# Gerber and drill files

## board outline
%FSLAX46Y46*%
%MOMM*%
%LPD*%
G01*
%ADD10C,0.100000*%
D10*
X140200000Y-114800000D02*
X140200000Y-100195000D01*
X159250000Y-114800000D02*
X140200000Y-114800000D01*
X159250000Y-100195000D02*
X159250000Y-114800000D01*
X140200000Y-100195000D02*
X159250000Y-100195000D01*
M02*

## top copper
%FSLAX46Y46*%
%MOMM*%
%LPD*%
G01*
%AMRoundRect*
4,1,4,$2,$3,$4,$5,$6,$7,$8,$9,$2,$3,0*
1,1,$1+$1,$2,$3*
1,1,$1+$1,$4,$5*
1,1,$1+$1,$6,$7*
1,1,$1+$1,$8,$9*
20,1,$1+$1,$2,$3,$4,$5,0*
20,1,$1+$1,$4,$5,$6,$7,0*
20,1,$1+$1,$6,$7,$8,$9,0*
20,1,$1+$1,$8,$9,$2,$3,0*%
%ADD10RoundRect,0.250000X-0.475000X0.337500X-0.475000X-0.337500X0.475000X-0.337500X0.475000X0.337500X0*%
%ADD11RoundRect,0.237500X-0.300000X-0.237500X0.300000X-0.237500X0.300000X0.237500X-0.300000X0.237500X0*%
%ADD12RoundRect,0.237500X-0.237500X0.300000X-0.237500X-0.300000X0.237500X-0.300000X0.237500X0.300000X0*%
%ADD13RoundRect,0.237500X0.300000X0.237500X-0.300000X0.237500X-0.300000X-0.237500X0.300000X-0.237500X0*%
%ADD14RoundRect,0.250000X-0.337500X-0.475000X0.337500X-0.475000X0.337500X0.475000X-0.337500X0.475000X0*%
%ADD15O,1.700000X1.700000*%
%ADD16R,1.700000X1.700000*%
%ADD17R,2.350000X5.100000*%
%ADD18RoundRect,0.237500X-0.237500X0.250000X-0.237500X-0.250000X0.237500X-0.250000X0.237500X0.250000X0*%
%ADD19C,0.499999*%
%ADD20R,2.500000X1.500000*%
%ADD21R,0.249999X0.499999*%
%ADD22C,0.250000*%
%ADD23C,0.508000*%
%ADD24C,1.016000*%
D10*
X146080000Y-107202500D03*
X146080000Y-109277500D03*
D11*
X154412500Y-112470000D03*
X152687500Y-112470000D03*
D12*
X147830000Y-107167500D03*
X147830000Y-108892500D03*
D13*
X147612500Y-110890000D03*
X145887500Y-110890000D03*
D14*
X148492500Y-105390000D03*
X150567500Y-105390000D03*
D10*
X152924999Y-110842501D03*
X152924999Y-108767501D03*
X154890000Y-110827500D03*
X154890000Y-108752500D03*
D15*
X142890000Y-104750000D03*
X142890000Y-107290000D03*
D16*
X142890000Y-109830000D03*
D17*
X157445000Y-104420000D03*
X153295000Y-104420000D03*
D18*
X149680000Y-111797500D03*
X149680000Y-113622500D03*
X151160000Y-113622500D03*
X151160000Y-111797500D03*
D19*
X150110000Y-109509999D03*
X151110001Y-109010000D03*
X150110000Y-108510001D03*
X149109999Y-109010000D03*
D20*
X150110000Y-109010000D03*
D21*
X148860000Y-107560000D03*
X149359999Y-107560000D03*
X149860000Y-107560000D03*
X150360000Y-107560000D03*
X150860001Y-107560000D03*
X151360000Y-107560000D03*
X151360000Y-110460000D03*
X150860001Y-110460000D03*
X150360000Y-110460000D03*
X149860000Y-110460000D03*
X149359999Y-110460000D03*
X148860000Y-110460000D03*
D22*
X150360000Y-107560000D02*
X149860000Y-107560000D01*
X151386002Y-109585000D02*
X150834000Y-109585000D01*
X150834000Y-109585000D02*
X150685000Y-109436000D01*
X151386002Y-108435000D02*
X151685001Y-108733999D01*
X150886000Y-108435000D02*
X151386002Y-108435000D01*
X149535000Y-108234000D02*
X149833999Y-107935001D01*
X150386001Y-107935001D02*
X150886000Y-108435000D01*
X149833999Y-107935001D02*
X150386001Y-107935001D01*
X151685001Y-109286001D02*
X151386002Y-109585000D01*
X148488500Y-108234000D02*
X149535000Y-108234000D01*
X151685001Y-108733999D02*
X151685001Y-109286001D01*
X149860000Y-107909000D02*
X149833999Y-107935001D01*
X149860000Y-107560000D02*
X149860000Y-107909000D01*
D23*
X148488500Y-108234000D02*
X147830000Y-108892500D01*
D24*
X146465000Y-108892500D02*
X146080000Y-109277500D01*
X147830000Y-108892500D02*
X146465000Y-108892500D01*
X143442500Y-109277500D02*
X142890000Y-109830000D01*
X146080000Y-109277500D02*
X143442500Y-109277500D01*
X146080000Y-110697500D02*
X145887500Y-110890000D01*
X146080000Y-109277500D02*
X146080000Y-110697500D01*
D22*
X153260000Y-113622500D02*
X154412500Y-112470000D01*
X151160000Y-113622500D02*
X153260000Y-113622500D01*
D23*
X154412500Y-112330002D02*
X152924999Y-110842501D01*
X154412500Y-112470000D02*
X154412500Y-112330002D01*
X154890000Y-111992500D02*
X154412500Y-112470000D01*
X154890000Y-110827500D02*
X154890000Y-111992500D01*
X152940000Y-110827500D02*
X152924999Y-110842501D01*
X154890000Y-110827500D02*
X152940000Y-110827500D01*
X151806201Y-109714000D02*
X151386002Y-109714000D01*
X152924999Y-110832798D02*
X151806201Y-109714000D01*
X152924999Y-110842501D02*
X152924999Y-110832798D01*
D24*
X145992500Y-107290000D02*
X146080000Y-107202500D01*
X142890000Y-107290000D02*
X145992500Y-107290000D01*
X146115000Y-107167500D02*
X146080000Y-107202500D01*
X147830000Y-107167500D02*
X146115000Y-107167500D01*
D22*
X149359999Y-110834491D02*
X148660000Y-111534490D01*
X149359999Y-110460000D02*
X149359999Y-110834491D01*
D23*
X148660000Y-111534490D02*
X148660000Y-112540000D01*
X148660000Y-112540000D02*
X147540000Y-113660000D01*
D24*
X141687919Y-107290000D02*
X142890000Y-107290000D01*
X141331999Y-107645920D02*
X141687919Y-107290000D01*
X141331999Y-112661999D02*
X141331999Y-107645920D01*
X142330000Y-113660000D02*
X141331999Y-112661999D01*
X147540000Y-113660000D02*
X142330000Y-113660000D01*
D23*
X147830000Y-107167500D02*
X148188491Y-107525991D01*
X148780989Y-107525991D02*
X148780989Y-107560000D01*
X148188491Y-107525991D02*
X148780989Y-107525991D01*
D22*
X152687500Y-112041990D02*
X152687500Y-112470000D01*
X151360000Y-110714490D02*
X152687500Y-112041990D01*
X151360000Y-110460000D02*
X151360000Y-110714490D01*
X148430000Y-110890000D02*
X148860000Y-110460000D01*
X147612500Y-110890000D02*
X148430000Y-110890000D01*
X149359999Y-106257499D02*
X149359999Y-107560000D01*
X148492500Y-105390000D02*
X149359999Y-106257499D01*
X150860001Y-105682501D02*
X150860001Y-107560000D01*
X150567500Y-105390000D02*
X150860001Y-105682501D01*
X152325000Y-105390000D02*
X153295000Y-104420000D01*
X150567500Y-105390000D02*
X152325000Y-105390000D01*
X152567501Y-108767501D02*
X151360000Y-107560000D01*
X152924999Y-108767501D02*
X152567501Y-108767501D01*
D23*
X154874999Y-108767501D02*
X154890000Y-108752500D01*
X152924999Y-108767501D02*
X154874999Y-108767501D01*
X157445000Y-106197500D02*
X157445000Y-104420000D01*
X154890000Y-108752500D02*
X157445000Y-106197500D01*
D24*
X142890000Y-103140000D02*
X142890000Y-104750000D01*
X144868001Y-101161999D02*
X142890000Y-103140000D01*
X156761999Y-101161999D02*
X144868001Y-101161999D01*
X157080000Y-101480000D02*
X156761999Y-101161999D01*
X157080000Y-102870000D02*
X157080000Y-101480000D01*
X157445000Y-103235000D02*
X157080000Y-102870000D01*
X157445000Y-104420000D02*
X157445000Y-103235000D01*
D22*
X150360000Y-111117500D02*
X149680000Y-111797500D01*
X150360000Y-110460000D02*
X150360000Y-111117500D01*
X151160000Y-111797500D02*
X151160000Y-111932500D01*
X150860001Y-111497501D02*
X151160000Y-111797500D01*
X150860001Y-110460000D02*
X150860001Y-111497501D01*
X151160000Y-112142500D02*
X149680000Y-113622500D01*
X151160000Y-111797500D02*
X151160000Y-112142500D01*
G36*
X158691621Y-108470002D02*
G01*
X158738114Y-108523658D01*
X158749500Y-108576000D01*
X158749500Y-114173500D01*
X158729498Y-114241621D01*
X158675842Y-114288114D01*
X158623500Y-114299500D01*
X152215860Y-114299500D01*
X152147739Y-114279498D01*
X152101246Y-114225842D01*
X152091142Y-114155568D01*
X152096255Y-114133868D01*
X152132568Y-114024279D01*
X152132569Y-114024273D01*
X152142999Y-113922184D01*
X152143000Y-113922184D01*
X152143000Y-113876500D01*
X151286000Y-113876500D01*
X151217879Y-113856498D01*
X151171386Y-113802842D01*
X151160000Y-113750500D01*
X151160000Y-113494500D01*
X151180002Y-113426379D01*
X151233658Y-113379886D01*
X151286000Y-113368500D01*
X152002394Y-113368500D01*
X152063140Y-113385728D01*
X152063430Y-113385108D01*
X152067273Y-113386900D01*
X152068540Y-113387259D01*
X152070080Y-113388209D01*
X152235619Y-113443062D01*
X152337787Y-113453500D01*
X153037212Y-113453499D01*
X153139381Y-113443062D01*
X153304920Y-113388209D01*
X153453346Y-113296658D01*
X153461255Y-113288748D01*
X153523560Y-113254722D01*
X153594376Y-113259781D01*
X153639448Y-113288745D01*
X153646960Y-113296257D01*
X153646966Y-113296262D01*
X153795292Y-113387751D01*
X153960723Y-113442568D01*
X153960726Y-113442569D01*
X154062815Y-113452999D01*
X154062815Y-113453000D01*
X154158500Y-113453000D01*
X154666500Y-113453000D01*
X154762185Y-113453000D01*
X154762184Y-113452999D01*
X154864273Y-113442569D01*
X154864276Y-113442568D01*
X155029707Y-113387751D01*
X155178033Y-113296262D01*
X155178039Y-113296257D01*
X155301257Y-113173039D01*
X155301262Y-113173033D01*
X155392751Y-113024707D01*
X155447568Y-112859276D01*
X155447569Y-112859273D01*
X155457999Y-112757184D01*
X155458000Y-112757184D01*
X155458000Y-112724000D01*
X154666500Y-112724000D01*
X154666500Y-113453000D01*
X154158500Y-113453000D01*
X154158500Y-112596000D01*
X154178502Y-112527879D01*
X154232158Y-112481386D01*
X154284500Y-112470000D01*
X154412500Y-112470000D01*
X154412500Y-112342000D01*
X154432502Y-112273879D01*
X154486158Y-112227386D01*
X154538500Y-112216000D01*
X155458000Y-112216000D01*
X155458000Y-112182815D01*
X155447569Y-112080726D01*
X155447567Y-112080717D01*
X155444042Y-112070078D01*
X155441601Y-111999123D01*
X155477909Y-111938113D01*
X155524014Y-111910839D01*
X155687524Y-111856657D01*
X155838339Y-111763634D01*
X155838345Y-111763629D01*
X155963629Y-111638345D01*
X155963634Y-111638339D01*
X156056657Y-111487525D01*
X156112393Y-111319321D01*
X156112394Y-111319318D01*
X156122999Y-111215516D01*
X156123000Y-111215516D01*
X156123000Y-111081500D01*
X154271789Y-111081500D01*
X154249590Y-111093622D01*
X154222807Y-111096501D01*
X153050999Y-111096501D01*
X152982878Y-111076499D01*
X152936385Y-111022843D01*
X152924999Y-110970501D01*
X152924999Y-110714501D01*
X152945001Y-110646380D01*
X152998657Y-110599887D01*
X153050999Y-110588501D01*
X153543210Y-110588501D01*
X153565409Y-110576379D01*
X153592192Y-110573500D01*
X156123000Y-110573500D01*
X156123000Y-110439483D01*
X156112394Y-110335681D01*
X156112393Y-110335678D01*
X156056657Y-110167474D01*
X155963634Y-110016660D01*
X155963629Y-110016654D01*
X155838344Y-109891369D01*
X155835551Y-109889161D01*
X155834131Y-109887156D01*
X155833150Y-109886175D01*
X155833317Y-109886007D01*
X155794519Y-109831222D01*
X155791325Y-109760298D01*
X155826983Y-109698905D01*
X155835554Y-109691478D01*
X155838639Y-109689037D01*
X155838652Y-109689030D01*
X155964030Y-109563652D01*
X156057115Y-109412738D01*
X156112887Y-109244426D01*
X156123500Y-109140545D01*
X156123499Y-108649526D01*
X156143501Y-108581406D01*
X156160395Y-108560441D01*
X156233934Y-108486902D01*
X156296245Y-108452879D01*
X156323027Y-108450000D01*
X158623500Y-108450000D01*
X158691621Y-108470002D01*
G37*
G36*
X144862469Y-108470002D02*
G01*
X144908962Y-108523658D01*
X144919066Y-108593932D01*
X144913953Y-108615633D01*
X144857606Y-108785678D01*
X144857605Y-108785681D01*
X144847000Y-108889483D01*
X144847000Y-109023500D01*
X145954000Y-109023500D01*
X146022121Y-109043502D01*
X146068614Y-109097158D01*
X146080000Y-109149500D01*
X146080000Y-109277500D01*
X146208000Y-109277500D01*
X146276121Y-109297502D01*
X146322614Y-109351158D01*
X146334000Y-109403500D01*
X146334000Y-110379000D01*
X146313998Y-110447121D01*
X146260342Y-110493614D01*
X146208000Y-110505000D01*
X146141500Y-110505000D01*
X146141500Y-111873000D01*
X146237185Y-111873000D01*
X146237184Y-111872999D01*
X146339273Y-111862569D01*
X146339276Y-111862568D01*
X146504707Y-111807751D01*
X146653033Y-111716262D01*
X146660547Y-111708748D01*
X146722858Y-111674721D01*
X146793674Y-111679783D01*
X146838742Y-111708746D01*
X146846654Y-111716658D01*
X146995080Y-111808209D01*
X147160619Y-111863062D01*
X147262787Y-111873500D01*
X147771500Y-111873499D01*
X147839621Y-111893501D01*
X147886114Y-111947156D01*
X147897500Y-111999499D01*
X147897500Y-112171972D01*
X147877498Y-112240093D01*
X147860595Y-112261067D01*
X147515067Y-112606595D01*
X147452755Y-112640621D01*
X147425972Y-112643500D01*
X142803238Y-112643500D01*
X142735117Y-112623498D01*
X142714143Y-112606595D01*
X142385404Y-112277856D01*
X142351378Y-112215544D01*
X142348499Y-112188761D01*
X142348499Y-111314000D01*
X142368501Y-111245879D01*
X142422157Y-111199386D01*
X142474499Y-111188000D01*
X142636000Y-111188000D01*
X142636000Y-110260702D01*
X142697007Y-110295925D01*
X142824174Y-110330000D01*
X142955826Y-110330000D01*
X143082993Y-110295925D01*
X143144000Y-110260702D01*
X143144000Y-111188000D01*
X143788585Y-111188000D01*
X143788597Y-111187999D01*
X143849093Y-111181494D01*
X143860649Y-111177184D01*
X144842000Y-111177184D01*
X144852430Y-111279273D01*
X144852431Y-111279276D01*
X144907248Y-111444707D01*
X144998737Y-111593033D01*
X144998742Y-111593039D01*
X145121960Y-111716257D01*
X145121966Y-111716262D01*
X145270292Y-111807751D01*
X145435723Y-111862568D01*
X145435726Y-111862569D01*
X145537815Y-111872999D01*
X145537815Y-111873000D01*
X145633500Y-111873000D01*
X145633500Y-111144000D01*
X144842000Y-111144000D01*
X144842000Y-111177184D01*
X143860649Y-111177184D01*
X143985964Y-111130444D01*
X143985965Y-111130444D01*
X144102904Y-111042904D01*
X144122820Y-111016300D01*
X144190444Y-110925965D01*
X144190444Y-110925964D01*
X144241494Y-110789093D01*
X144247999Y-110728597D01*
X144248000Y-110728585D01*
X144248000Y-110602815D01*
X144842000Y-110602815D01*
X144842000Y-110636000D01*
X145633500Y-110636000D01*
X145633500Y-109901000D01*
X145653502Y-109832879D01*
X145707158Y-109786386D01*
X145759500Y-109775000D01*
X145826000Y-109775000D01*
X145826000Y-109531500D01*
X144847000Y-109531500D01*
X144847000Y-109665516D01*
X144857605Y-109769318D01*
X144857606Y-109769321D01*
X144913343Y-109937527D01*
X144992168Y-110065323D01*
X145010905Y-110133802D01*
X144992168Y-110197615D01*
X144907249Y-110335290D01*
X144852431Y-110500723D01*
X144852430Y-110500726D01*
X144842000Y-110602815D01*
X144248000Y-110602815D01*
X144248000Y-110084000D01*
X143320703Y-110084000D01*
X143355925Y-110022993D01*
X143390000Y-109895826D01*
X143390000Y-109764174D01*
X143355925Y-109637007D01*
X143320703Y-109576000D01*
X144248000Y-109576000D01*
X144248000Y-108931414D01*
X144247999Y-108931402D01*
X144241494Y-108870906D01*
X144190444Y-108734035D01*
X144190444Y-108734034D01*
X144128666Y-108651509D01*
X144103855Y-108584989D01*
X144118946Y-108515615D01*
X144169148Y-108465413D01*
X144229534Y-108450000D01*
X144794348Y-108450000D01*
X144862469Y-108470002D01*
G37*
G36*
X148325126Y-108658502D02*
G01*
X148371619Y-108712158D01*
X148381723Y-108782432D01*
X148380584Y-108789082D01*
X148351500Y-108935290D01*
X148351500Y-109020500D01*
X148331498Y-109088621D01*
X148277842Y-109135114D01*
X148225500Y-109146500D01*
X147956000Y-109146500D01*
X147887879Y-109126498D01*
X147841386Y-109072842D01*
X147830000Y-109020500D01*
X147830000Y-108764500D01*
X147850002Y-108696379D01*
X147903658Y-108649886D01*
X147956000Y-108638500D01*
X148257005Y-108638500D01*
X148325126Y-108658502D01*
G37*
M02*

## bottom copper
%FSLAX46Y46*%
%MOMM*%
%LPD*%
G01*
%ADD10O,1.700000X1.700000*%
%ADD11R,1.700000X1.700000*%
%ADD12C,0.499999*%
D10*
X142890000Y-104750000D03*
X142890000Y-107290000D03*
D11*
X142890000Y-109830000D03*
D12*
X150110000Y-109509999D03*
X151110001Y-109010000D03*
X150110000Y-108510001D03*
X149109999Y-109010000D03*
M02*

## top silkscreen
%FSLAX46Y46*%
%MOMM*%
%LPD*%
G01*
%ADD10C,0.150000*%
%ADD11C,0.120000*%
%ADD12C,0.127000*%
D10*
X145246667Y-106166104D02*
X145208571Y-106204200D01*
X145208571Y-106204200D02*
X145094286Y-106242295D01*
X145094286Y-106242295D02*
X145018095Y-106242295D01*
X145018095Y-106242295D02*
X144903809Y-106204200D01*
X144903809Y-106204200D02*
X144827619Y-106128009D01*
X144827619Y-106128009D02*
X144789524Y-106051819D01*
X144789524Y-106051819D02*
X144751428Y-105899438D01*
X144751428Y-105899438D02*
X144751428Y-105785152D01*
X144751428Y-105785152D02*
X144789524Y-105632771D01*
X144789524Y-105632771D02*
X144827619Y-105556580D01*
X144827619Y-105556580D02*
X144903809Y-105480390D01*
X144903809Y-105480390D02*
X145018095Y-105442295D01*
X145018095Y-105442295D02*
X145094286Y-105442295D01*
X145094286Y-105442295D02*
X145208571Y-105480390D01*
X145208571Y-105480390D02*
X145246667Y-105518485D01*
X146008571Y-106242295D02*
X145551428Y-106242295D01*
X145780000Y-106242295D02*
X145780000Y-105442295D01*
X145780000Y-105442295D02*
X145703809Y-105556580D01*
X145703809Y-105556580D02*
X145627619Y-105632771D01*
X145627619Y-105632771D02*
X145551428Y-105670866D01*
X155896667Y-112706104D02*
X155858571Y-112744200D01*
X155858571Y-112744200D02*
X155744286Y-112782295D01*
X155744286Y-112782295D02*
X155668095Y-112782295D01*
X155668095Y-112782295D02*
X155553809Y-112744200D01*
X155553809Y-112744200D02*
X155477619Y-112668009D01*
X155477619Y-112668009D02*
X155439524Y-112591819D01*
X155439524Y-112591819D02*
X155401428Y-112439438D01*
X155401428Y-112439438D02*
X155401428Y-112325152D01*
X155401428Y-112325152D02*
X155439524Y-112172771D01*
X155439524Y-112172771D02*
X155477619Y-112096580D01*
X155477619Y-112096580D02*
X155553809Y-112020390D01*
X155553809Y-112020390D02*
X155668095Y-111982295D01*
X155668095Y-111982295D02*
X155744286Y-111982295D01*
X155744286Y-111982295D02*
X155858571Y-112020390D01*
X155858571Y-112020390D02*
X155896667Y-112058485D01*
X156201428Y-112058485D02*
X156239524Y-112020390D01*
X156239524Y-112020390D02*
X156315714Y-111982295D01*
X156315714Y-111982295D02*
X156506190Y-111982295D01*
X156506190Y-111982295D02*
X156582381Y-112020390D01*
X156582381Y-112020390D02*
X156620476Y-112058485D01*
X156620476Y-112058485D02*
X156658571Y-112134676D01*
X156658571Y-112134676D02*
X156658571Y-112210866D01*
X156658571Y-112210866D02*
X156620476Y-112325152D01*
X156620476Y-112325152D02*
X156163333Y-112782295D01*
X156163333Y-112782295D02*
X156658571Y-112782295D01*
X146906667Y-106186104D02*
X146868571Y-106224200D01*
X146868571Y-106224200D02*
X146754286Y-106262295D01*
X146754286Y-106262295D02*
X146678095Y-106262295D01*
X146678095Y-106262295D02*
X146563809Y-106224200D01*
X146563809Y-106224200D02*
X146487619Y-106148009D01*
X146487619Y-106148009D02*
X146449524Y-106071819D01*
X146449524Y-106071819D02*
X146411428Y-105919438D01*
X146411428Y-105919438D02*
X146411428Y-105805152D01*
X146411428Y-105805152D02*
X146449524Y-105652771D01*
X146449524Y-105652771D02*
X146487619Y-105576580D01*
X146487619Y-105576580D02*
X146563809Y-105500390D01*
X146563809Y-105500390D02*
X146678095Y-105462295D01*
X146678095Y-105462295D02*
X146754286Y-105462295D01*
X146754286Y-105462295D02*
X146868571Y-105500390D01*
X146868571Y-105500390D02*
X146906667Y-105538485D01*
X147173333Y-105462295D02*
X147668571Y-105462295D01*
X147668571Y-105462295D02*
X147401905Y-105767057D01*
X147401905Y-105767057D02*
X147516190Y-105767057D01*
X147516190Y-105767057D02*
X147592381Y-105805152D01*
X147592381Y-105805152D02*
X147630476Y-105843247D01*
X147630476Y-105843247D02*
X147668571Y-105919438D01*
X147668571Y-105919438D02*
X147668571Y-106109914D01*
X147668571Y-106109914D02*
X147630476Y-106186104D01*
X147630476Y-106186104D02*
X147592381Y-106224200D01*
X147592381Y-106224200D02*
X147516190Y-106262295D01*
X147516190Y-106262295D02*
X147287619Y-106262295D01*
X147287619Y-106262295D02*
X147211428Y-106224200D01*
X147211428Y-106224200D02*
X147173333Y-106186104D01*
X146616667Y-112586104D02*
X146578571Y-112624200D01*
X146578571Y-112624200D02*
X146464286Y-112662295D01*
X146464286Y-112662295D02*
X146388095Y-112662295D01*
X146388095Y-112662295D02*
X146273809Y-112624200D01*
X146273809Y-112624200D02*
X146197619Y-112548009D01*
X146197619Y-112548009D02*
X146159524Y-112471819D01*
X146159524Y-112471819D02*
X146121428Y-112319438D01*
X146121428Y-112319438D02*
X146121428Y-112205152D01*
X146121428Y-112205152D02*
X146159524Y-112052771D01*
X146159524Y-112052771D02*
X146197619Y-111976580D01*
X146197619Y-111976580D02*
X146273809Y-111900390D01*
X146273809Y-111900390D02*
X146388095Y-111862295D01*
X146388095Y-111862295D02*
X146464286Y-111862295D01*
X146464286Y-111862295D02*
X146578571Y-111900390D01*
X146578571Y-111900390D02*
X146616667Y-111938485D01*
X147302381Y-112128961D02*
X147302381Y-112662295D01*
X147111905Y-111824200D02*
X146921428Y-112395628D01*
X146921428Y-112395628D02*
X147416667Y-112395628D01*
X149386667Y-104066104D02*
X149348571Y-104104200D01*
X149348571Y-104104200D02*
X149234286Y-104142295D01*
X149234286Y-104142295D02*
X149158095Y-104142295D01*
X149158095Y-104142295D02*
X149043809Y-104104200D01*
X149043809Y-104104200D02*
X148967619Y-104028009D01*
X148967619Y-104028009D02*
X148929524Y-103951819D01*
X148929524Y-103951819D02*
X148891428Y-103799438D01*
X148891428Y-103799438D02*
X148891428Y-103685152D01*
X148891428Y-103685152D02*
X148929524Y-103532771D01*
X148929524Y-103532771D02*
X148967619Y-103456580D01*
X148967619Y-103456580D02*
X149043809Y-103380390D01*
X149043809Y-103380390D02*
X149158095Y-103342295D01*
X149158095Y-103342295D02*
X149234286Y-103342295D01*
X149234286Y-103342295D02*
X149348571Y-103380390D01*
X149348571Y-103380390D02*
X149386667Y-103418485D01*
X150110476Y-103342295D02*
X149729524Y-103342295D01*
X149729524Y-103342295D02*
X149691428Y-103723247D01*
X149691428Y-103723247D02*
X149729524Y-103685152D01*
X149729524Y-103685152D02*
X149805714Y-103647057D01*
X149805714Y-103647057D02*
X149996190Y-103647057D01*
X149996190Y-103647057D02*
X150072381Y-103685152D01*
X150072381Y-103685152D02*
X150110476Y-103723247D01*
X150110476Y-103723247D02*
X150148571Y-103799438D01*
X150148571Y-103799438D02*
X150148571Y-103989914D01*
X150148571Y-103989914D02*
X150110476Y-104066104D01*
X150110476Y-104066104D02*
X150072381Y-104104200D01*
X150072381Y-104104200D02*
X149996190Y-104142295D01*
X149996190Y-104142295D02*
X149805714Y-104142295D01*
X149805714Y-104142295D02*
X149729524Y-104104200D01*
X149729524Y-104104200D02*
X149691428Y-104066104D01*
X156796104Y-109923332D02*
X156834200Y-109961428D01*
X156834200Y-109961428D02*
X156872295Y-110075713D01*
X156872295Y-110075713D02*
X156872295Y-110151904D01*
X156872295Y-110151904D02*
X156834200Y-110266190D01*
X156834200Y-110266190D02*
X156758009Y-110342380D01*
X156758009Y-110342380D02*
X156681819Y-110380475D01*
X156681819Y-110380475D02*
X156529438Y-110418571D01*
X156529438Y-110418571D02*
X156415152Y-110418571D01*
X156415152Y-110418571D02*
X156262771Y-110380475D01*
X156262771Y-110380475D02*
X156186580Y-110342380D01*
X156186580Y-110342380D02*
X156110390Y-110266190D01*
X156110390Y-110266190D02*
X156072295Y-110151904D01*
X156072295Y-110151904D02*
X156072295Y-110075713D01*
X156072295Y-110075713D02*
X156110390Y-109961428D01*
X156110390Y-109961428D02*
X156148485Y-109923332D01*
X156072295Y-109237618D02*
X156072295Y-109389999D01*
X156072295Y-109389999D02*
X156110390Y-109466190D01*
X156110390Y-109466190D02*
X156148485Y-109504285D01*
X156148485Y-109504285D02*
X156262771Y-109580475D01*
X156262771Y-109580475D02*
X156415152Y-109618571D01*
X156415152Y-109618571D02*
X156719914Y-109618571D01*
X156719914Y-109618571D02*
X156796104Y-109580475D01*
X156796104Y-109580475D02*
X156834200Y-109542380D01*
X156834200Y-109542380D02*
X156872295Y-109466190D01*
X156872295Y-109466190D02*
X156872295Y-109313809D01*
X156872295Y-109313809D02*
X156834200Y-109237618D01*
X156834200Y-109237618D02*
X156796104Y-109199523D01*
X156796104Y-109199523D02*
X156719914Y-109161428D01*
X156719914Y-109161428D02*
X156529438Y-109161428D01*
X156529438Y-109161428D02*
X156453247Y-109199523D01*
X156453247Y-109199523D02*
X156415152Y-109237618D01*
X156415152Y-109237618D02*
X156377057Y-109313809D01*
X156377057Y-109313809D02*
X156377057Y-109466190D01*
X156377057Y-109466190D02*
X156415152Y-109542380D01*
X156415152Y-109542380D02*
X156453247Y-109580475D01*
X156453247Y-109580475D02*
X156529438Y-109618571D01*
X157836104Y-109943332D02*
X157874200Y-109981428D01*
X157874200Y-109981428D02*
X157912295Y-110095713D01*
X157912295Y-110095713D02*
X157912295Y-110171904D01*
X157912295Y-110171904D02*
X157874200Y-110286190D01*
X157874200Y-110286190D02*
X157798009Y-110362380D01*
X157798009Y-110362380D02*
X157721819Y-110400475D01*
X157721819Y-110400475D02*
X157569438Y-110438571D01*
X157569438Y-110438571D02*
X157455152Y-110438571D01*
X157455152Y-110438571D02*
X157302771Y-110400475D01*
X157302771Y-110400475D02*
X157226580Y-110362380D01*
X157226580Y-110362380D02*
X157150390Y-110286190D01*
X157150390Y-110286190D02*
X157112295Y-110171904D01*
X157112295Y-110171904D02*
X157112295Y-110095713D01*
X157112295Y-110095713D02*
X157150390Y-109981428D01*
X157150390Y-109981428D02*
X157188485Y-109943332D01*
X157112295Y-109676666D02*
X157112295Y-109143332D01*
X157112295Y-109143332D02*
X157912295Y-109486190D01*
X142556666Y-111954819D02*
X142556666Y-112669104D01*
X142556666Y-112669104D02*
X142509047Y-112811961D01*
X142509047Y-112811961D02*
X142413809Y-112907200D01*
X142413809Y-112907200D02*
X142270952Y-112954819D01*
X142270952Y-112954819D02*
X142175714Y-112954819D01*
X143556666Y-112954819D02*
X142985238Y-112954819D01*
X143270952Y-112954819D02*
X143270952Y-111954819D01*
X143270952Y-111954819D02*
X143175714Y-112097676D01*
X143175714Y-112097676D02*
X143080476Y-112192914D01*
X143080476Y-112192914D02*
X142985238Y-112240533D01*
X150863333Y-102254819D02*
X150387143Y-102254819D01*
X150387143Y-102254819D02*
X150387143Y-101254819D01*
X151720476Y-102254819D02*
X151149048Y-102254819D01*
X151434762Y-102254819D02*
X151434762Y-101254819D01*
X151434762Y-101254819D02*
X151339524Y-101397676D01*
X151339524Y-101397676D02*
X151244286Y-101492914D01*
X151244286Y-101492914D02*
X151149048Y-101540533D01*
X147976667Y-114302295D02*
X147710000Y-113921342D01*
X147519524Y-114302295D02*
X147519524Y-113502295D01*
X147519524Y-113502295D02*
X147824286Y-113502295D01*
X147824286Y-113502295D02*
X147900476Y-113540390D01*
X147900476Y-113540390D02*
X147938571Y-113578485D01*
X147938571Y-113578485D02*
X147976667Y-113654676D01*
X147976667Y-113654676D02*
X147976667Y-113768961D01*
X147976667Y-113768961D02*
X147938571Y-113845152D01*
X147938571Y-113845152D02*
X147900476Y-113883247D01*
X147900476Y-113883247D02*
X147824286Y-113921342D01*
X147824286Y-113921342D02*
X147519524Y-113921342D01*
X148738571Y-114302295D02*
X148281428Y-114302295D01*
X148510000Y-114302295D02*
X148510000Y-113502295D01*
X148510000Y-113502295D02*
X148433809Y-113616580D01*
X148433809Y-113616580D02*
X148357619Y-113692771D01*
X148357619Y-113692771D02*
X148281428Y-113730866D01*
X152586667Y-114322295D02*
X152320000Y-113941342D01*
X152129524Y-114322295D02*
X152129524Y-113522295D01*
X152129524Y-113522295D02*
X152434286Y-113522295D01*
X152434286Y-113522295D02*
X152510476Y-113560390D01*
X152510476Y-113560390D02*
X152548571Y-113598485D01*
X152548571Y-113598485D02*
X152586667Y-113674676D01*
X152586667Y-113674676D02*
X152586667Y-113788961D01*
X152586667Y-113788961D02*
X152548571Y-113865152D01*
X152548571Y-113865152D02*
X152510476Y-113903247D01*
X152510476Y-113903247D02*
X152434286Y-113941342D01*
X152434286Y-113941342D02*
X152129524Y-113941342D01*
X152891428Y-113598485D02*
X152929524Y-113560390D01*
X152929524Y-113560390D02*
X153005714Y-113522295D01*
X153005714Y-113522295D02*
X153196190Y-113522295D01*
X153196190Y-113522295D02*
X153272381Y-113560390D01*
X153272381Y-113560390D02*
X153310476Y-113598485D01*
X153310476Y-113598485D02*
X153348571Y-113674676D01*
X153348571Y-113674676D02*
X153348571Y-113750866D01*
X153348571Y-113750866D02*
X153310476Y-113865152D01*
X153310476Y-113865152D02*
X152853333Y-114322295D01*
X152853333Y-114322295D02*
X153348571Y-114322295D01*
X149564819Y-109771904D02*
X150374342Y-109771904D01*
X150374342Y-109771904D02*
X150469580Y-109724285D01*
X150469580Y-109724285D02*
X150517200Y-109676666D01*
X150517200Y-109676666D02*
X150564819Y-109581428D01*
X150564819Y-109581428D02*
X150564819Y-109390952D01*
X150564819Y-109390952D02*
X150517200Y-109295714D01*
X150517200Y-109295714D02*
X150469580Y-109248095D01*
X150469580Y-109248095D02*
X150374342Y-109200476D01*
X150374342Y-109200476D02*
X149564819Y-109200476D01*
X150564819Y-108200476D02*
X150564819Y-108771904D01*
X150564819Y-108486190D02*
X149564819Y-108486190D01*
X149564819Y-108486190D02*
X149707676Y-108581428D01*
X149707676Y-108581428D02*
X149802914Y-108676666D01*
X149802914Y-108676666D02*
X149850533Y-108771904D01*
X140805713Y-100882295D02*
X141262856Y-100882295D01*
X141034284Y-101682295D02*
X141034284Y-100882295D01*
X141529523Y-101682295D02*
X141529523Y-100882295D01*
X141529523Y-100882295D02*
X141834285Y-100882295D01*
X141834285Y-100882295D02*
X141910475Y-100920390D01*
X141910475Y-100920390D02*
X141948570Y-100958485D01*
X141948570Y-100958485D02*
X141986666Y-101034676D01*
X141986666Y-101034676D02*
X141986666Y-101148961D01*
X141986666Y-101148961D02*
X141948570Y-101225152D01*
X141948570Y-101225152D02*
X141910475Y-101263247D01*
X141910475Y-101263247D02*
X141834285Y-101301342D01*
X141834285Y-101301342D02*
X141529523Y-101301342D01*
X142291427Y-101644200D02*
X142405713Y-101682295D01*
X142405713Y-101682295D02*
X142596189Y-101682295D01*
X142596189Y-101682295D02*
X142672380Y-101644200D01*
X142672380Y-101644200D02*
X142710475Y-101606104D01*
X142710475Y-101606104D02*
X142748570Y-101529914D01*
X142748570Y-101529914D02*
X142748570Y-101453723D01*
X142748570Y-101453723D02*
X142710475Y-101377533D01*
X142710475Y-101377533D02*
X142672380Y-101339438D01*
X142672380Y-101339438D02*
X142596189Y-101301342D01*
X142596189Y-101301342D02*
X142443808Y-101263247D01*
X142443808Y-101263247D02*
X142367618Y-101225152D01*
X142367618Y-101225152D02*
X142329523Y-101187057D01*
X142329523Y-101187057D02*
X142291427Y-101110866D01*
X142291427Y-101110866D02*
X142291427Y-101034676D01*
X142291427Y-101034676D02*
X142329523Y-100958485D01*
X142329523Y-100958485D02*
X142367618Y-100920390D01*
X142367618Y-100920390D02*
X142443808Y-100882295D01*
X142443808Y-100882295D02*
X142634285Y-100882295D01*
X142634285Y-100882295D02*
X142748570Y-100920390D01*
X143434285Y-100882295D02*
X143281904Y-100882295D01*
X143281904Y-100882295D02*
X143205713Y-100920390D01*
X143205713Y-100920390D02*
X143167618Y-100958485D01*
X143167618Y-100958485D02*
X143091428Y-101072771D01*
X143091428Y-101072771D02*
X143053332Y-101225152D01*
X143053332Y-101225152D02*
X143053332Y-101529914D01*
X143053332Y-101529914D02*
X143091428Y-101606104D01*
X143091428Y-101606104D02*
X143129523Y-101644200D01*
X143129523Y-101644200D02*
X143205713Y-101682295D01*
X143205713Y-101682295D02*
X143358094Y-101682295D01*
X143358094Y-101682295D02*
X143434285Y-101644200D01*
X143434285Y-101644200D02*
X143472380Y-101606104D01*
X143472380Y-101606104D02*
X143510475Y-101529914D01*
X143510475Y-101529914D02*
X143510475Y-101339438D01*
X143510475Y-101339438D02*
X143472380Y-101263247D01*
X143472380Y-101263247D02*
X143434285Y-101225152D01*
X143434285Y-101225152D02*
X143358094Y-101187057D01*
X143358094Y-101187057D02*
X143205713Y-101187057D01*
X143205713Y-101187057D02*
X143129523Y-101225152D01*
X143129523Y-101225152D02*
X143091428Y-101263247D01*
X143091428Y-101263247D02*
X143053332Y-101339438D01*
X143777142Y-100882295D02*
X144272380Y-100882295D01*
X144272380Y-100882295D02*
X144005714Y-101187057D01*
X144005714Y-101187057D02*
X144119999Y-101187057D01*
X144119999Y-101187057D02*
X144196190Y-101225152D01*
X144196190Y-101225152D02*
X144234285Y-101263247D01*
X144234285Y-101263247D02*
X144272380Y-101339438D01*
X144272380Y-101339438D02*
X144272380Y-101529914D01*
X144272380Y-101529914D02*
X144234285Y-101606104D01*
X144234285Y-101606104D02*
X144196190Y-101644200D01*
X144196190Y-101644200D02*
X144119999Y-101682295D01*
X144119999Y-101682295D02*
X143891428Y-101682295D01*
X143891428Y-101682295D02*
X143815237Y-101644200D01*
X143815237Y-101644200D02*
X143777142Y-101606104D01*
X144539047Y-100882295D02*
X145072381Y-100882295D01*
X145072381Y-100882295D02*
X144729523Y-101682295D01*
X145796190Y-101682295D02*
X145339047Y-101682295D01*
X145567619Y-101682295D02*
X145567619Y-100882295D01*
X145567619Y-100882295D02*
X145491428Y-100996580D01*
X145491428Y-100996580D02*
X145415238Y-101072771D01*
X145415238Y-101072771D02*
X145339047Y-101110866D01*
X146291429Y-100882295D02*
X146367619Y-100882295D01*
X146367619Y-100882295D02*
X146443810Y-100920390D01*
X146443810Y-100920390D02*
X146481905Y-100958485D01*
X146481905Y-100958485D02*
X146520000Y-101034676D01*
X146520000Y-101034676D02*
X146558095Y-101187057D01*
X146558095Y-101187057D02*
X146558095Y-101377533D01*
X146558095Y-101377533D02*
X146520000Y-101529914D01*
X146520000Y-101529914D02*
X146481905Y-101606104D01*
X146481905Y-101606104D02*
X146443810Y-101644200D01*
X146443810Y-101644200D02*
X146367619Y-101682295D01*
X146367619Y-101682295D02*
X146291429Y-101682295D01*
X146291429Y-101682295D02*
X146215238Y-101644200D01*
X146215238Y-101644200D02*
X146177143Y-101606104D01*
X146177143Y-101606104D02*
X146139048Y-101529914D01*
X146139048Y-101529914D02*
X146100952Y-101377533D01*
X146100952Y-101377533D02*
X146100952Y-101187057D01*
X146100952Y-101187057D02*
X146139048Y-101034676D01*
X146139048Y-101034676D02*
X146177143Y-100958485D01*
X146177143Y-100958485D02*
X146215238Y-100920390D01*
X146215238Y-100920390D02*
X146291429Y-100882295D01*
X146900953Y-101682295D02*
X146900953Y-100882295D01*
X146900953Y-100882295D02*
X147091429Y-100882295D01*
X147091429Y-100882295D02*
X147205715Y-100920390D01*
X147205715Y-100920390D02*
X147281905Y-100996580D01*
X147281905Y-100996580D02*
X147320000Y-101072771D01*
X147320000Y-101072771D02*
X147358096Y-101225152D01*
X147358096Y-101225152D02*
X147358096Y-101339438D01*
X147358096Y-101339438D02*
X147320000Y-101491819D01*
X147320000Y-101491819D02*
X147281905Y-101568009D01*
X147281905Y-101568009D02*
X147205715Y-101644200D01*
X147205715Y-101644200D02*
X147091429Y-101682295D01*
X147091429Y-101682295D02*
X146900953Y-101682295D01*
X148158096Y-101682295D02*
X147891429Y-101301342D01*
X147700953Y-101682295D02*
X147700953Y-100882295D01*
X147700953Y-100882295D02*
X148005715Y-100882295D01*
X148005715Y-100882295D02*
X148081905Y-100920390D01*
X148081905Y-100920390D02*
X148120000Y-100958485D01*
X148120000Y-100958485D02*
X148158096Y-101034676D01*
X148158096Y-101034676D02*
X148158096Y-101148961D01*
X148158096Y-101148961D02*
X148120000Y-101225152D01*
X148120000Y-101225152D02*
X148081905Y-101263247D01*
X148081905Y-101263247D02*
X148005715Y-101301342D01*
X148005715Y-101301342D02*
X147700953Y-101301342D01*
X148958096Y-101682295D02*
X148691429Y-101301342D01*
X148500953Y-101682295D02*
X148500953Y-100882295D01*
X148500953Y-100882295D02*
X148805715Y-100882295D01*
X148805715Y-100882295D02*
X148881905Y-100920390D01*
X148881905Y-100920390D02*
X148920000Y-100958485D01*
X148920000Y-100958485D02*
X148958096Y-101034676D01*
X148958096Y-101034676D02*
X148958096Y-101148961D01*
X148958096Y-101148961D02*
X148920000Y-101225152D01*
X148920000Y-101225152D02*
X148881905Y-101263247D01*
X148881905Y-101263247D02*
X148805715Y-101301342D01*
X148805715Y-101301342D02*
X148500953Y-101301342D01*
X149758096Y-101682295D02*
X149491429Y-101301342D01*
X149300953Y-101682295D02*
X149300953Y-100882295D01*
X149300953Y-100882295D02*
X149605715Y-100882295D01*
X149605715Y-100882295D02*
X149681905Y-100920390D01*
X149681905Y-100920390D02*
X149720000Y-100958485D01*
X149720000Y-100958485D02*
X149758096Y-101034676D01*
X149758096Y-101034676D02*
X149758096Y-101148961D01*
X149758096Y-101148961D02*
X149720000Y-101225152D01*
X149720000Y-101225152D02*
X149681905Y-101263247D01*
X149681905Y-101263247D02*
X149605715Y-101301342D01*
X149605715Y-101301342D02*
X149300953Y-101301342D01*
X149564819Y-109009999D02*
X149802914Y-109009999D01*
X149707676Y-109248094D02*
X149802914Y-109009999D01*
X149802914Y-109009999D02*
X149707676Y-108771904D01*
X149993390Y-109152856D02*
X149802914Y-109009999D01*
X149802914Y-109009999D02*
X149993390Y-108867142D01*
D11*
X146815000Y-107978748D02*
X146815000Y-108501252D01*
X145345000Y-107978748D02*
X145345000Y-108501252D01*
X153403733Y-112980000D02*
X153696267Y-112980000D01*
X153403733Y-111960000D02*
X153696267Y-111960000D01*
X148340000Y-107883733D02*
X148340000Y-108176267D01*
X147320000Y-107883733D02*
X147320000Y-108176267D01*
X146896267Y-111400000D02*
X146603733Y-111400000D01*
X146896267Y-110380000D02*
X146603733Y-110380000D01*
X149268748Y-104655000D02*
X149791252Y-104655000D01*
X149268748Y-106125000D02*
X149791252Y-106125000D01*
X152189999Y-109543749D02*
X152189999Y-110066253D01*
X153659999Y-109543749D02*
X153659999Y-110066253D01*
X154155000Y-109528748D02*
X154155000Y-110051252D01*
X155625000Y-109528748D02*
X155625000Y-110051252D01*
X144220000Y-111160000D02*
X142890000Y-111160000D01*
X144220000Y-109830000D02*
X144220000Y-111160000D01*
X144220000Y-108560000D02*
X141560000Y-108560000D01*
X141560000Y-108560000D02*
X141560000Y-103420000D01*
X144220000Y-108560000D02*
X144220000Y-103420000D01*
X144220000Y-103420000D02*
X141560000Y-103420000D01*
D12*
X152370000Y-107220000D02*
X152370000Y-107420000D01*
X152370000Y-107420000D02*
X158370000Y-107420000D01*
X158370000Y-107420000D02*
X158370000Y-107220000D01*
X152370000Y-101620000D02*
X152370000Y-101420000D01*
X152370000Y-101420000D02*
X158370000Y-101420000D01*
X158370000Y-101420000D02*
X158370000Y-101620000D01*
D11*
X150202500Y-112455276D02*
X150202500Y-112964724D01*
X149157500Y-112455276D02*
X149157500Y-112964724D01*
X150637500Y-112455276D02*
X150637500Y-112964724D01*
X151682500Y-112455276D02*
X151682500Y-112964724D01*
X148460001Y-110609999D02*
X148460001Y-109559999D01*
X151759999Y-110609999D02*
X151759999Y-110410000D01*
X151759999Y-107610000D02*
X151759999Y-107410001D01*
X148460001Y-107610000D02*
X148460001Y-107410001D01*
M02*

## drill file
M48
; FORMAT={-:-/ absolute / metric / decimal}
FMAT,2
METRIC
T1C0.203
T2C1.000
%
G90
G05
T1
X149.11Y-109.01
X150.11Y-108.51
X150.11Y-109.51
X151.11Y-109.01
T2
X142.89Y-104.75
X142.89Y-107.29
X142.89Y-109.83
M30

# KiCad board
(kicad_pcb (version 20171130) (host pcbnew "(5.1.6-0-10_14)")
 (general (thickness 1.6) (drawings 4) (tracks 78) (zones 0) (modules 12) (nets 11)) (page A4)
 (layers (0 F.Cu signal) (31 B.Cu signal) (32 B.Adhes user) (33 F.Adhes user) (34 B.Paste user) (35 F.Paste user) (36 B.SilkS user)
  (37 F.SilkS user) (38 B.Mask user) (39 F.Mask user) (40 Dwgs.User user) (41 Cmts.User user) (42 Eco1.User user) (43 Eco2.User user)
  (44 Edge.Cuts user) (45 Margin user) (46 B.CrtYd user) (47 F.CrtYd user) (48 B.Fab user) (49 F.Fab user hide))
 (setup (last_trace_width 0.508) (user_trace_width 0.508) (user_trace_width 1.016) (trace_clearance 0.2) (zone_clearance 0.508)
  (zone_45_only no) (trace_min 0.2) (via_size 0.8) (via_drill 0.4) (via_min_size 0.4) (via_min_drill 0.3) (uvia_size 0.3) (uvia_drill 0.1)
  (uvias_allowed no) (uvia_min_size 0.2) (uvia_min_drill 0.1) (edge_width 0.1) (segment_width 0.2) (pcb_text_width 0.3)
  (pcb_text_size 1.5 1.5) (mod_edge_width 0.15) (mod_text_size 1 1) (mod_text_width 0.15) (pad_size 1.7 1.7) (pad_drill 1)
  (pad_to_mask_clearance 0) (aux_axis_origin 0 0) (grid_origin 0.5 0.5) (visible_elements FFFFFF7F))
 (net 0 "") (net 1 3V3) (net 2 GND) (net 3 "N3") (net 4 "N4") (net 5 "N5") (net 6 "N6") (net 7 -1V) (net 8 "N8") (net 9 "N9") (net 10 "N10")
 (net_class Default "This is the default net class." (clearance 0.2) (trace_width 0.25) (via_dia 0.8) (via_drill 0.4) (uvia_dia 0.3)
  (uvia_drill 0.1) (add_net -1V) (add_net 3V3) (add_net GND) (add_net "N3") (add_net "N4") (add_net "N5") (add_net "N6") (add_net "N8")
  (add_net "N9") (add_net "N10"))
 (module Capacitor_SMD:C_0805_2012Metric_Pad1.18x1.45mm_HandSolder (layer F.Cu) (at 146.08 108.24 270)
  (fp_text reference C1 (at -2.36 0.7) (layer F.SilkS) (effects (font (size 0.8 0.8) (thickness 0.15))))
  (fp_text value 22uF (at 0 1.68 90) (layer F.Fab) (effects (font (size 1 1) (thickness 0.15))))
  (fp_line (start -0.261252 -0.735) (end 0.261252 -0.735) (layer F.SilkS) (width 0.12))
  (fp_line (start -0.261252 0.735) (end 0.261252 0.735) (layer F.SilkS) (width 0.12))
  (pad 1 smd roundrect (at -1.0375 0 270) (size 1.175 1.45) (layers F.Cu F.Paste F.Mask) (roundrect_rratio 0.212766) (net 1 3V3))
  (pad 2 smd roundrect (at 1.0375 0 270) (size 1.175 1.45) (layers F.Cu F.Paste F.Mask) (roundrect_rratio 0.212766) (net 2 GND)))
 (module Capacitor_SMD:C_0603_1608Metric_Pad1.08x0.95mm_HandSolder (layer F.Cu) (at 153.55 112.47)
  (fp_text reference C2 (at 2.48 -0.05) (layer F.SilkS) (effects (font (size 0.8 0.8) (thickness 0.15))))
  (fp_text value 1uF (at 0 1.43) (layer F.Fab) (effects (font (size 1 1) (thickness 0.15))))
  (fp_line (start -0.146267 0.51) (end 0.146267 0.51) (layer F.SilkS) (width 0.12))
  (fp_line (start -0.146267 -0.51) (end 0.146267 -0.51) (layer F.SilkS) (width 0.12))
  (pad 2 smd roundrect (at 0.8625 0) (size 1.075 0.95) (layers F.Cu F.Paste F.Mask) (roundrect_rratio 0.25) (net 2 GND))
  (pad 1 smd roundrect (at -0.8625 0) (size 1.075 0.95) (layers F.Cu F.Paste F.Mask) (roundrect_rratio 0.25) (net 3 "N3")))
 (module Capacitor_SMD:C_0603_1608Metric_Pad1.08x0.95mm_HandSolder (layer F.Cu) (at 147.83 108.03 270)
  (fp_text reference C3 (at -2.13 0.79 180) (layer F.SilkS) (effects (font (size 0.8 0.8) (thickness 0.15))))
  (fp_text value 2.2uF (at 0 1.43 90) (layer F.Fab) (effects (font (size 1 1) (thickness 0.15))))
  (fp_line (start -0.146267 -0.51) (end 0.146267 -0.51) (layer F.SilkS) (width 0.12))
  (fp_line (start -0.146267 0.51) (end 0.146267 0.51) (layer F.SilkS) (width 0.12))
  (pad 1 smd roundrect (at -0.8625 0 270) (size 1.075 0.95) (layers F.Cu F.Paste F.Mask) (roundrect_rratio 0.25) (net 1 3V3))
  (pad 2 smd roundrect (at 0.8625 0 270) (size 1.075 0.95) (layers F.Cu F.Paste F.Mask) (roundrect_rratio 0.25) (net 2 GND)))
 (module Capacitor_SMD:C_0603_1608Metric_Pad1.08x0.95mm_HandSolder (layer F.Cu) (at 146.75 110.89 180)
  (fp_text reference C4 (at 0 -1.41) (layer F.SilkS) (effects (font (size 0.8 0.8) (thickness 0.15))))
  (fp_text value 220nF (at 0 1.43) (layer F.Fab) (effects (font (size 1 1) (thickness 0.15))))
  (fp_line (start -0.146267 -0.51) (end 0.146267 -0.51) (layer F.SilkS) (width 0.12))
  (fp_line (start -0.146267 0.51) (end 0.146267 0.51) (layer F.SilkS) (width 0.12))
  (pad 1 smd roundrect (at -0.8625 0 180) (size 1.075 0.95) (layers F.Cu F.Paste F.Mask) (roundrect_rratio 0.25) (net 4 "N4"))
  (pad 2 smd roundrect (at 0.8625 0 180) (size 1.075 0.95) (layers F.Cu F.Paste F.Mask) (roundrect_rratio 0.25) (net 2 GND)))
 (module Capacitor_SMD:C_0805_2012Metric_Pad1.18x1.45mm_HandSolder (layer F.Cu) (at 149.53 105.39)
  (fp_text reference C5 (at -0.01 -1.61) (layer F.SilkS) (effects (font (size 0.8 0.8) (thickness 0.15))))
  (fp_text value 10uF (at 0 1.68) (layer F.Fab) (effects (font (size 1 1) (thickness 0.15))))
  (fp_line (start -0.261252 -0.735) (end 0.261252 -0.735) (layer F.SilkS) (width 0.12))
  (fp_line (start -0.261252 0.735) (end 0.261252 0.735) (layer F.SilkS) (width 0.12))
  (pad 1 smd roundrect (at -1.0375 0) (size 1.175 1.45) (layers F.Cu F.Paste F.Mask) (roundrect_rratio 0.212766) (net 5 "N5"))
  (pad 2 smd roundrect (at 1.0375 0) (size 1.175 1.45) (layers F.Cu F.Paste F.Mask) (roundrect_rratio 0.212766) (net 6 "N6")))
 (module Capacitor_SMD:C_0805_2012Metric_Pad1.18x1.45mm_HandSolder (layer F.Cu) (at 152.924999 109.805001 270)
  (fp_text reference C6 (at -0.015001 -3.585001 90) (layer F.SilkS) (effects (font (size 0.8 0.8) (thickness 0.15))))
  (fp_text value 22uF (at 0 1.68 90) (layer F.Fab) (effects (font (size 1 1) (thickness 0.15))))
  (fp_line (start -0.261252 0.735) (end 0.261252 0.735) (layer F.SilkS) (width 0.12))
  (fp_line (start -0.261252 -0.735) (end 0.261252 -0.735) (layer F.SilkS) (width 0.12))
  (pad 2 smd roundrect (at 1.0375 0 270) (size 1.175 1.45) (layers F.Cu F.Paste F.Mask) (roundrect_rratio 0.212766) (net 2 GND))
  (pad 1 smd roundrect (at -1.0375 0 270) (size 1.175 1.45) (layers F.Cu F.Paste F.Mask) (roundrect_rratio 0.212766) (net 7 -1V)))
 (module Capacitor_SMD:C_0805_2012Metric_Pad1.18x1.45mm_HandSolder (layer F.Cu) (at 154.89 109.79 270)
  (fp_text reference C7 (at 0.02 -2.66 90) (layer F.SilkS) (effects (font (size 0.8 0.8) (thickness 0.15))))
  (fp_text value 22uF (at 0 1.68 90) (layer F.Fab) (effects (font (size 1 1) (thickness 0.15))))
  (fp_line (start -0.261252 0.735) (end 0.261252 0.735) (layer F.SilkS) (width 0.12))
  (fp_line (start -0.261252 -0.735) (end 0.261252 -0.735) (layer F.SilkS) (width 0.12))
  (pad 2 smd roundrect (at 1.0375 0 270) (size 1.175 1.45) (layers F.Cu F.Paste F.Mask) (roundrect_rratio 0.212766) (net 2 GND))
  (pad 1 smd roundrect (at -1.0375 0 270) (size 1.175 1.45) (layers F.Cu F.Paste F.Mask) (roundrect_rratio 0.212766) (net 7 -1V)))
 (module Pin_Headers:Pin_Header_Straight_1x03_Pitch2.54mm (layer F.Cu) (at 142.89 109.83 180)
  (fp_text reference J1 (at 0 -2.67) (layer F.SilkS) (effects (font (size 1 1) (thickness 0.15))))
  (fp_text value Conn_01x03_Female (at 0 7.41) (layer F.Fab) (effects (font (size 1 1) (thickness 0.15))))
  (fp_line (start -1.33 -1.33) (end 0 -1.33) (layer F.SilkS) (width 0.12))
  (fp_line (start -1.33 0) (end -1.33 -1.33) (layer F.SilkS) (width 0.12))
  (fp_line (start -1.33 1.27) (end 1.33 1.27) (layer F.SilkS) (width 0.12))
  (fp_line (start 1.33 1.27) (end 1.33 6.41) (layer F.SilkS) (width 0.12))
  (fp_line (start -1.33 1.27) (end -1.33 6.41) (layer F.SilkS) (width 0.12))
  (fp_line (start -1.33 6.41) (end 1.33 6.41) (layer F.SilkS) (width 0.12))
  (pad 3 thru_hole oval (at 0 5.08 180) (size 1.7 1.7) (drill 1) (layers *.Cu *.Mask) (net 7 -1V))
  (pad 2 thru_hole oval (at 0 2.54 180) (size 1.7 1.7) (drill 1) (layers *.Cu *.Mask) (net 1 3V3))
  (pad 1 thru_hole rect (at 0 0 180) (size 1.7 1.7) (drill 1) (layers *.Cu *.Mask) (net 2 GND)))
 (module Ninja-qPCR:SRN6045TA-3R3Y (layer F.Cu) (at 155.37 104.42)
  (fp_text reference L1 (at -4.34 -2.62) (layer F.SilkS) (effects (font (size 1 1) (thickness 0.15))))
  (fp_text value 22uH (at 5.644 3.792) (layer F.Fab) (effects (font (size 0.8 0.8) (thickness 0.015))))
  (fp_line (start -3 2.8) (end -3 3) (layer F.SilkS) (width 0.127))
  (fp_line (start -3 3) (end 3 3) (layer F.SilkS) (width 0.127))
  (fp_line (start 3 3) (end 3 2.8) (layer F.SilkS) (width 0.127))
  (fp_line (start -3 -2.8) (end -3 -3) (layer F.SilkS) (width 0.127))
  (fp_line (start -3 -3) (end 3 -3) (layer F.SilkS) (width 0.127))
  (fp_line (start 3 -3) (end 3 -2.8) (layer F.SilkS) (width 0.127))
  (pad 2 smd rect (at 2.075 0) (size 2.35 5.1) (layers F.Cu F.Paste F.Mask) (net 7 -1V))
  (pad 1 smd rect (at -2.075 0) (size 2.35 5.1) (layers F.Cu F.Paste F.Mask) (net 6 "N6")))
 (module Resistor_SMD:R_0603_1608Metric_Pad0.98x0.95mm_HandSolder (layer F.Cu) (at 149.68 112.71 270)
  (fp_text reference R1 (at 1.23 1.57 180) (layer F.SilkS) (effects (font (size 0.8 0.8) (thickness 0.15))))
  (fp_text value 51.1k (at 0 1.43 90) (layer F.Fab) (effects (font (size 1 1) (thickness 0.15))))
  (fp_line (start -0.254724 -0.5225) (end 0.254724 -0.5225) (layer F.SilkS) (width 0.12))
  (fp_line (start -0.254724 0.5225) (end 0.254724 0.5225) (layer F.SilkS) (width 0.12))
  (pad 1 smd roundrect (at -0.9125 0 270) (size 0.975 0.95) (layers F.Cu F.Paste F.Mask) (roundrect_rratio 0.25) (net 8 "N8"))
  (pad 2 smd roundrect (at 0.9125 0 270) (size 0.975 0.95) (layers F.Cu F.Paste F.Mask) (roundrect_rratio 0.25) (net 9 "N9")))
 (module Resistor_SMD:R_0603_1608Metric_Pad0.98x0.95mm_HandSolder (layer F.Cu) (at 151.16 112.71 270)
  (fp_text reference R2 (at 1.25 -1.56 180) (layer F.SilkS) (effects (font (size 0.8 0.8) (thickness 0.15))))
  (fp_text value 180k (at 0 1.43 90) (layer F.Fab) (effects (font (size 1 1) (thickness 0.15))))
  (fp_line (start -0.254724 0.5225) (end 0.254724 0.5225) (layer F.SilkS) (width 0.12))
  (fp_line (start -0.254724 -0.5225) (end 0.254724 -0.5225) (layer F.SilkS) (width 0.12))
  (pad 2 smd roundrect (at 0.9125 0 270) (size 0.975 0.95) (layers F.Cu F.Paste F.Mask) (roundrect_rratio 0.25) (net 2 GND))
  (pad 1 smd roundrect (at -0.9125 0 270) (size 0.975 0.95) (layers F.Cu F.Paste F.Mask) (roundrect_rratio 0.25) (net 9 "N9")))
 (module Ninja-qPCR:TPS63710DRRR (layer F.Cu) (at 150.11 109.01 90)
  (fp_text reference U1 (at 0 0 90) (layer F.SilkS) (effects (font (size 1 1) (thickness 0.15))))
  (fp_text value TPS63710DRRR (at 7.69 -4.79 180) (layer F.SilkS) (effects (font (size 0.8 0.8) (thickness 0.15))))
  (fp_line (start -1.599999 -1.649999) (end -0.549999 -1.649999) (layer F.SilkS) (width 0.12))
  (fp_line (start -1.599999 1.649999) (end -1.4 1.649999) (layer F.SilkS) (width 0.12))
  (fp_line (start 1.4 1.649999) (end 1.599999 1.649999) (layer F.SilkS) (width 0.12))
  (fp_line (start 1.4 -1.649999) (end 1.599999 -1.649999) (layer F.SilkS) (width 0.12))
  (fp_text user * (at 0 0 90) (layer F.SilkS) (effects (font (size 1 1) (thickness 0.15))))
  (pad V thru_hole circle (at -0.499999 0 90) (size 0.499999 0.499999) (drill 0.2032) (layers *.Cu *.Mask))
  (pad V thru_hole circle (at 0 1.000001 90) (size 0.499999 0.499999) (drill 0.2032) (layers *.Cu *.Mask))
  (pad V thru_hole circle (at 0.499999 0 90) (size 0.499999 0.499999) (drill 0.2032) (layers *.Cu *.Mask))
  (pad V thru_hole circle (at 0 -1.000001 90) (size 0.499999 0.499999) (drill 0.2032) (layers *.Cu *.Mask))
  (pad 13 smd rect (at 0 0 90) (size 1.5 2.5) (layers F.Cu F.Paste F.Mask) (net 2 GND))
  (pad 12 smd rect (at 1.45 -1.25 90) (size 0.499999 0.249999) (layers F.Cu F.Paste F.Mask) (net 1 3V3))
  (pad 11 smd rect (at 1.45 -0.750001 90) (size 0.499999 0.249999) (layers F.Cu F.Paste F.Mask) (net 5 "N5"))
  (pad 10 smd rect (at 1.45 -0.25 90) (size 0.499999 0.249999) (layers F.Cu F.Paste F.Mask) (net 2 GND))
  (pad 9 smd rect (at 1.45 0.25 90) (size 0.499999 0.249999) (layers F.Cu F.Paste F.Mask) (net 2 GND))
  (pad 8 smd rect (at 1.45 0.750001 90) (size 0.499999 0.249999) (layers F.Cu F.Paste F.Mask) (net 6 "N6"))
  (pad 7 smd rect (at 1.45 1.25 90) (size 0.499999 0.249999) (layers F.Cu F.Paste F.Mask) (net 7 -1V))
  (pad 6 smd rect (at -1.45 1.25 90) (size 0.499999 0.249999) (layers F.Cu F.Paste F.Mask) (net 3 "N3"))
  (pad 5 smd rect (at -1.45 0.750001 90) (size 0.499999 0.249999) (layers F.Cu F.Paste F.Mask) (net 9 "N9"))
  (pad 4 smd rect (at -1.45 0.25 90) (size 0.499999 0.249999) (layers F.Cu F.Paste F.Mask) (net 8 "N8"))
  (pad 3 smd rect (at -1.45 -0.25 90) (size 0.499999 0.249999) (layers F.Cu F.Paste F.Mask) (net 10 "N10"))
  (pad 2 smd rect (at -1.45 -0.750001 90) (size 0.499999 0.249999) (layers F.Cu F.Paste F.Mask) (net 1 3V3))
  (pad 1 smd rect (at -1.45 -1.25 90) (size 0.499999 0.249999) (layers F.Cu F.Paste F.Mask) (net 4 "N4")))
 (gr_line (start 140.2 114.8) (end 140.2 100.195) (layer Edge.Cuts) (width 0.1))
 (gr_line (start 159.25 114.8) (end 140.2 114.8) (layer Edge.Cuts) (width 0.1))
 (gr_line (start 159.25 100.195) (end 159.25 114.8) (layer Edge.Cuts) (width 0.1))
 (gr_line (start 140.2 100.195) (end 159.25 100.195) (layer Edge.Cuts) (width 0.1))
 (segment (start 150.36 107.56) (end 149.86 107.56) (width 0.25) (layer F.Cu) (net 2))
 (segment (start 151.386002 109.585) (end 150.834 109.585) (width 0.25) (layer F.Cu) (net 2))
 (segment (start 150.834 109.585) (end 150.685 109.436) (width 0.25) (layer F.Cu) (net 2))
 (segment (start 151.386002 108.435) (end 151.685001 108.733999) (width 0.25) (layer F.Cu) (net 2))
 (segment (start 150.886 108.435) (end 151.386002 108.435) (width 0.25) (layer F.Cu) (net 2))
 (segment (start 149.535 108.234) (end 149.833999 107.935001) (width 0.25) (layer F.Cu) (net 2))
 (segment (start 150.386001 107.935001) (end 150.886 108.435) (width 0.25) (layer F.Cu) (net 2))
 (segment (start 149.833999 107.935001) (end 150.386001 107.935001) (width 0.25) (layer F.Cu) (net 2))
 (segment (start 151.685001 109.286001) (end 151.386002 109.585) (width 0.25) (layer F.Cu) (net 2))
 (segment (start 148.4885 108.234) (end 149.535 108.234) (width 0.25) (layer F.Cu) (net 2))
 (segment (start 151.685001 108.733999) (end 151.685001 109.286001) (width 0.25) (layer F.Cu) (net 2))
 (segment (start 149.86 107.909) (end 149.833999 107.935001) (width 0.25) (layer F.Cu) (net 2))
 (segment (start 149.86 107.56) (end 149.86 107.909) (width 0.25) (layer F.Cu) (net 2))
 (segment (start 148.4885 108.234) (end 147.83 108.8925) (width 0.508) (layer F.Cu) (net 2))
 (segment (start 146.465 108.8925) (end 146.08 109.2775) (width 1.016) (layer F.Cu) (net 2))
 (segment (start 147.83 108.8925) (end 146.465 108.8925) (width 1.016) (layer F.Cu) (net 2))
 (segment (start 143.4425 109.2775) (end 142.89 109.83) (width 1.016) (layer F.Cu) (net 2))
 (segment (start 146.08 109.2775) (end 143.4425 109.2775) (width 1.016) (layer F.Cu) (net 2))
 (segment (start 146.08 110.6975) (end 145.8875 110.89) (width 1.016) (layer F.Cu) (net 2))
 (segment (start 146.08 109.2775) (end 146.08 110.6975) (width 1.016) (layer F.Cu) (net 2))
 (segment (start 153.26 113.6225) (end 154.4125 112.47) (width 0.25) (layer F.Cu) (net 2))
 (segment (start 151.16 113.6225) (end 153.26 113.6225) (width 0.25) (layer F.Cu) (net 2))
 (segment (start 154.4125 112.330002) (end 152.924999 110.842501) (width 0.508) (layer F.Cu) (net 2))
 (segment (start 154.4125 112.47) (end 154.4125 112.330002) (width 0.508) (layer F.Cu) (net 2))
 (segment (start 154.89 111.9925) (end 154.4125 112.47) (width 0.508) (layer F.Cu) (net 2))
 (segment (start 154.89 110.8275) (end 154.89 111.9925) (width 0.508) (layer F.Cu) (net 2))
 (segment (start 152.94 110.8275) (end 152.924999 110.842501) (width 0.508) (layer F.Cu) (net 2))
 (segment (start 154.89 110.8275) (end 152.94 110.8275) (width 0.508) (layer F.Cu) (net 2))
 (segment (start 151.806201 109.714) (end 151.386002 109.714) (width 0.508) (layer F.Cu) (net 2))
 (segment (start 152.924999 110.832798) (end 151.806201 109.714) (width 0.508) (layer F.Cu) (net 2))
 (segment (start 152.924999 110.842501) (end 152.924999 110.832798) (width 0.508) (layer F.Cu) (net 2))
 (segment (start 145.9925 107.29) (end 146.08 107.2025) (width 1.016) (layer F.Cu) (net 1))
 (segment (start 142.89 107.29) (end 145.9925 107.29) (width 1.016) (layer F.Cu) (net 1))
 (segment (start 146.115 107.1675) (end 146.08 107.2025) (width 1.016) (layer F.Cu) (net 1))
 (segment (start 147.83 107.1675) (end 146.115 107.1675) (width 1.016) (layer F.Cu) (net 1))
 (segment (start 149.359999 110.834491) (end 148.66 111.53449) (width 0.25) (layer F.Cu) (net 1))
 (segment (start 149.359999 110.46) (end 149.359999 110.834491) (width 0.25) (layer F.Cu) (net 1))
 (segment (start 148.66 111.53449) (end 148.66 112.54) (width 0.508) (layer F.Cu) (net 1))
 (segment (start 148.66 112.54) (end 147.54 113.66) (width 0.508) (layer F.Cu) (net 1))
 (segment (start 141.687919 107.29) (end 142.89 107.29) (width 1.016) (layer F.Cu) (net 1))
 (segment (start 141.331999 107.64592) (end 141.687919 107.29) (width 1.016) (layer F.Cu) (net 1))
 (segment (start 141.331999 112.661999) (end 141.331999 107.64592) (width 1.016) (layer F.Cu) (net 1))
 (segment (start 142.33 113.66) (end 141.331999 112.661999) (width 1.016) (layer F.Cu) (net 1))
 (segment (start 147.54 113.66) (end 142.33 113.66) (width 1.016) (layer F.Cu) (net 1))
 (segment (start 147.83 107.1675) (end 148.188491 107.525991) (width 0.508) (layer F.Cu) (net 1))
 (segment (start 148.780989 107.525991) (end 148.780989 107.56) (width 0.508) (layer F.Cu) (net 1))
 (segment (start 148.188491 107.525991) (end 148.780989 107.525991) (width 0.508) (layer F.Cu) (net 1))
 (segment (start 152.6875 112.04199) (end 152.6875 112.47) (width 0.25) (layer F.Cu) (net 3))
 (segment (start 151.36 110.71449) (end 152.6875 112.04199) (width 0.25) (layer F.Cu) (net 3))
 (segment (start 151.36 110.46) (end 151.36 110.71449) (width 0.25) (layer F.Cu) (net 3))
 (segment (start 148.43 110.89) (end 148.86 110.46) (width 0.25) (layer F.Cu) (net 4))
 (segment (start 147.6125 110.89) (end 148.43 110.89) (width 0.25) (layer F.Cu) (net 4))
 (segment (start 149.359999 106.257499) (end 149.359999 107.56) (width 0.25) (layer F.Cu) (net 5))
 (segment (start 148.4925 105.39) (end 149.359999 106.257499) (width 0.25) (layer F.Cu) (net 5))
 (segment (start 150.860001 105.682501) (end 150.860001 107.56) (width 0.25) (layer F.Cu) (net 6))
 (segment (start 150.5675 105.39) (end 150.860001 105.682501) (width 0.25) (layer F.Cu) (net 6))
 (segment (start 152.325 105.39) (end 153.295 104.42) (width 0.25) (layer F.Cu) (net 6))
 (segment (start 150.5675 105.39) (end 152.325 105.39) (width 0.25) (layer F.Cu) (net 6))
 (segment (start 152.567501 108.767501) (end 151.36 107.56) (width 0.25) (layer F.Cu) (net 7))
 (segment (start 152.924999 108.767501) (end 152.567501 108.767501) (width 0.25) (layer F.Cu) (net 7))
 (segment (start 154.874999 108.767501) (end 154.89 108.7525) (width 0.508) (layer F.Cu) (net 7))
 (segment (start 152.924999 108.767501) (end 154.874999 108.767501) (width 0.508) (layer F.Cu) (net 7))
 (segment (start 157.445 106.1975) (end 157.445 104.42) (width 0.508) (layer F.Cu) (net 7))
 (segment (start 154.89 108.7525) (end 157.445 106.1975) (width 0.508) (layer F.Cu) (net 7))
 (segment (start 142.89 103.14) (end 142.89 104.75) (width 1.016) (layer F.Cu) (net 7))
 (segment (start 144.868001 101.161999) (end 142.89 103.14) (width 1.016) (layer F.Cu) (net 7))
 (segment (start 156.761999 101.161999) (end 144.868001 101.161999) (width 1.016) (layer F.Cu) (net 7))
 (segment (start 157.08 101.48) (end 156.761999 101.161999) (width 1.016) (layer F.Cu) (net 7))
 (segment (start 157.08 102.87) (end 157.08 101.48) (width 1.016) (layer F.Cu) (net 7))
 (segment (start 157.445 103.235) (end 157.08 102.87) (width 1.016) (layer F.Cu) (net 7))
 (segment (start 157.445 104.42) (end 157.445 103.235) (width 1.016) (layer F.Cu) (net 7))
 (segment (start 150.36 111.1175) (end 149.68 111.7975) (width 0.25) (layer F.Cu) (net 8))
 (segment (start 150.36 110.46) (end 150.36 111.1175) (width 0.25) (layer F.Cu) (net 8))
 (segment (start 151.16 111.7975) (end 151.16 111.9325) (width 0.25) (layer F.Cu) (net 9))
 (segment (start 150.860001 111.497501) (end 151.16 111.7975) (width 0.25) (layer F.Cu) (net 9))
 (segment (start 150.860001 110.46) (end 150.860001 111.497501) (width 0.25) (layer F.Cu) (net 9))
 (segment (start 151.16 112.1425) (end 149.68 113.6225) (width 0.25) (layer F.Cu) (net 9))
 (segment (start 151.16 111.7975) (end 151.16 112.1425) (width 0.25) (layer F.Cu) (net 9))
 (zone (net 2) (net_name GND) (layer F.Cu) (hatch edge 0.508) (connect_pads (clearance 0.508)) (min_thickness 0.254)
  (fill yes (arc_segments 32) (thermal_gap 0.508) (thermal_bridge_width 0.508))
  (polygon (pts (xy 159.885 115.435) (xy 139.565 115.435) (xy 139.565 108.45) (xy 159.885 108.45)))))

